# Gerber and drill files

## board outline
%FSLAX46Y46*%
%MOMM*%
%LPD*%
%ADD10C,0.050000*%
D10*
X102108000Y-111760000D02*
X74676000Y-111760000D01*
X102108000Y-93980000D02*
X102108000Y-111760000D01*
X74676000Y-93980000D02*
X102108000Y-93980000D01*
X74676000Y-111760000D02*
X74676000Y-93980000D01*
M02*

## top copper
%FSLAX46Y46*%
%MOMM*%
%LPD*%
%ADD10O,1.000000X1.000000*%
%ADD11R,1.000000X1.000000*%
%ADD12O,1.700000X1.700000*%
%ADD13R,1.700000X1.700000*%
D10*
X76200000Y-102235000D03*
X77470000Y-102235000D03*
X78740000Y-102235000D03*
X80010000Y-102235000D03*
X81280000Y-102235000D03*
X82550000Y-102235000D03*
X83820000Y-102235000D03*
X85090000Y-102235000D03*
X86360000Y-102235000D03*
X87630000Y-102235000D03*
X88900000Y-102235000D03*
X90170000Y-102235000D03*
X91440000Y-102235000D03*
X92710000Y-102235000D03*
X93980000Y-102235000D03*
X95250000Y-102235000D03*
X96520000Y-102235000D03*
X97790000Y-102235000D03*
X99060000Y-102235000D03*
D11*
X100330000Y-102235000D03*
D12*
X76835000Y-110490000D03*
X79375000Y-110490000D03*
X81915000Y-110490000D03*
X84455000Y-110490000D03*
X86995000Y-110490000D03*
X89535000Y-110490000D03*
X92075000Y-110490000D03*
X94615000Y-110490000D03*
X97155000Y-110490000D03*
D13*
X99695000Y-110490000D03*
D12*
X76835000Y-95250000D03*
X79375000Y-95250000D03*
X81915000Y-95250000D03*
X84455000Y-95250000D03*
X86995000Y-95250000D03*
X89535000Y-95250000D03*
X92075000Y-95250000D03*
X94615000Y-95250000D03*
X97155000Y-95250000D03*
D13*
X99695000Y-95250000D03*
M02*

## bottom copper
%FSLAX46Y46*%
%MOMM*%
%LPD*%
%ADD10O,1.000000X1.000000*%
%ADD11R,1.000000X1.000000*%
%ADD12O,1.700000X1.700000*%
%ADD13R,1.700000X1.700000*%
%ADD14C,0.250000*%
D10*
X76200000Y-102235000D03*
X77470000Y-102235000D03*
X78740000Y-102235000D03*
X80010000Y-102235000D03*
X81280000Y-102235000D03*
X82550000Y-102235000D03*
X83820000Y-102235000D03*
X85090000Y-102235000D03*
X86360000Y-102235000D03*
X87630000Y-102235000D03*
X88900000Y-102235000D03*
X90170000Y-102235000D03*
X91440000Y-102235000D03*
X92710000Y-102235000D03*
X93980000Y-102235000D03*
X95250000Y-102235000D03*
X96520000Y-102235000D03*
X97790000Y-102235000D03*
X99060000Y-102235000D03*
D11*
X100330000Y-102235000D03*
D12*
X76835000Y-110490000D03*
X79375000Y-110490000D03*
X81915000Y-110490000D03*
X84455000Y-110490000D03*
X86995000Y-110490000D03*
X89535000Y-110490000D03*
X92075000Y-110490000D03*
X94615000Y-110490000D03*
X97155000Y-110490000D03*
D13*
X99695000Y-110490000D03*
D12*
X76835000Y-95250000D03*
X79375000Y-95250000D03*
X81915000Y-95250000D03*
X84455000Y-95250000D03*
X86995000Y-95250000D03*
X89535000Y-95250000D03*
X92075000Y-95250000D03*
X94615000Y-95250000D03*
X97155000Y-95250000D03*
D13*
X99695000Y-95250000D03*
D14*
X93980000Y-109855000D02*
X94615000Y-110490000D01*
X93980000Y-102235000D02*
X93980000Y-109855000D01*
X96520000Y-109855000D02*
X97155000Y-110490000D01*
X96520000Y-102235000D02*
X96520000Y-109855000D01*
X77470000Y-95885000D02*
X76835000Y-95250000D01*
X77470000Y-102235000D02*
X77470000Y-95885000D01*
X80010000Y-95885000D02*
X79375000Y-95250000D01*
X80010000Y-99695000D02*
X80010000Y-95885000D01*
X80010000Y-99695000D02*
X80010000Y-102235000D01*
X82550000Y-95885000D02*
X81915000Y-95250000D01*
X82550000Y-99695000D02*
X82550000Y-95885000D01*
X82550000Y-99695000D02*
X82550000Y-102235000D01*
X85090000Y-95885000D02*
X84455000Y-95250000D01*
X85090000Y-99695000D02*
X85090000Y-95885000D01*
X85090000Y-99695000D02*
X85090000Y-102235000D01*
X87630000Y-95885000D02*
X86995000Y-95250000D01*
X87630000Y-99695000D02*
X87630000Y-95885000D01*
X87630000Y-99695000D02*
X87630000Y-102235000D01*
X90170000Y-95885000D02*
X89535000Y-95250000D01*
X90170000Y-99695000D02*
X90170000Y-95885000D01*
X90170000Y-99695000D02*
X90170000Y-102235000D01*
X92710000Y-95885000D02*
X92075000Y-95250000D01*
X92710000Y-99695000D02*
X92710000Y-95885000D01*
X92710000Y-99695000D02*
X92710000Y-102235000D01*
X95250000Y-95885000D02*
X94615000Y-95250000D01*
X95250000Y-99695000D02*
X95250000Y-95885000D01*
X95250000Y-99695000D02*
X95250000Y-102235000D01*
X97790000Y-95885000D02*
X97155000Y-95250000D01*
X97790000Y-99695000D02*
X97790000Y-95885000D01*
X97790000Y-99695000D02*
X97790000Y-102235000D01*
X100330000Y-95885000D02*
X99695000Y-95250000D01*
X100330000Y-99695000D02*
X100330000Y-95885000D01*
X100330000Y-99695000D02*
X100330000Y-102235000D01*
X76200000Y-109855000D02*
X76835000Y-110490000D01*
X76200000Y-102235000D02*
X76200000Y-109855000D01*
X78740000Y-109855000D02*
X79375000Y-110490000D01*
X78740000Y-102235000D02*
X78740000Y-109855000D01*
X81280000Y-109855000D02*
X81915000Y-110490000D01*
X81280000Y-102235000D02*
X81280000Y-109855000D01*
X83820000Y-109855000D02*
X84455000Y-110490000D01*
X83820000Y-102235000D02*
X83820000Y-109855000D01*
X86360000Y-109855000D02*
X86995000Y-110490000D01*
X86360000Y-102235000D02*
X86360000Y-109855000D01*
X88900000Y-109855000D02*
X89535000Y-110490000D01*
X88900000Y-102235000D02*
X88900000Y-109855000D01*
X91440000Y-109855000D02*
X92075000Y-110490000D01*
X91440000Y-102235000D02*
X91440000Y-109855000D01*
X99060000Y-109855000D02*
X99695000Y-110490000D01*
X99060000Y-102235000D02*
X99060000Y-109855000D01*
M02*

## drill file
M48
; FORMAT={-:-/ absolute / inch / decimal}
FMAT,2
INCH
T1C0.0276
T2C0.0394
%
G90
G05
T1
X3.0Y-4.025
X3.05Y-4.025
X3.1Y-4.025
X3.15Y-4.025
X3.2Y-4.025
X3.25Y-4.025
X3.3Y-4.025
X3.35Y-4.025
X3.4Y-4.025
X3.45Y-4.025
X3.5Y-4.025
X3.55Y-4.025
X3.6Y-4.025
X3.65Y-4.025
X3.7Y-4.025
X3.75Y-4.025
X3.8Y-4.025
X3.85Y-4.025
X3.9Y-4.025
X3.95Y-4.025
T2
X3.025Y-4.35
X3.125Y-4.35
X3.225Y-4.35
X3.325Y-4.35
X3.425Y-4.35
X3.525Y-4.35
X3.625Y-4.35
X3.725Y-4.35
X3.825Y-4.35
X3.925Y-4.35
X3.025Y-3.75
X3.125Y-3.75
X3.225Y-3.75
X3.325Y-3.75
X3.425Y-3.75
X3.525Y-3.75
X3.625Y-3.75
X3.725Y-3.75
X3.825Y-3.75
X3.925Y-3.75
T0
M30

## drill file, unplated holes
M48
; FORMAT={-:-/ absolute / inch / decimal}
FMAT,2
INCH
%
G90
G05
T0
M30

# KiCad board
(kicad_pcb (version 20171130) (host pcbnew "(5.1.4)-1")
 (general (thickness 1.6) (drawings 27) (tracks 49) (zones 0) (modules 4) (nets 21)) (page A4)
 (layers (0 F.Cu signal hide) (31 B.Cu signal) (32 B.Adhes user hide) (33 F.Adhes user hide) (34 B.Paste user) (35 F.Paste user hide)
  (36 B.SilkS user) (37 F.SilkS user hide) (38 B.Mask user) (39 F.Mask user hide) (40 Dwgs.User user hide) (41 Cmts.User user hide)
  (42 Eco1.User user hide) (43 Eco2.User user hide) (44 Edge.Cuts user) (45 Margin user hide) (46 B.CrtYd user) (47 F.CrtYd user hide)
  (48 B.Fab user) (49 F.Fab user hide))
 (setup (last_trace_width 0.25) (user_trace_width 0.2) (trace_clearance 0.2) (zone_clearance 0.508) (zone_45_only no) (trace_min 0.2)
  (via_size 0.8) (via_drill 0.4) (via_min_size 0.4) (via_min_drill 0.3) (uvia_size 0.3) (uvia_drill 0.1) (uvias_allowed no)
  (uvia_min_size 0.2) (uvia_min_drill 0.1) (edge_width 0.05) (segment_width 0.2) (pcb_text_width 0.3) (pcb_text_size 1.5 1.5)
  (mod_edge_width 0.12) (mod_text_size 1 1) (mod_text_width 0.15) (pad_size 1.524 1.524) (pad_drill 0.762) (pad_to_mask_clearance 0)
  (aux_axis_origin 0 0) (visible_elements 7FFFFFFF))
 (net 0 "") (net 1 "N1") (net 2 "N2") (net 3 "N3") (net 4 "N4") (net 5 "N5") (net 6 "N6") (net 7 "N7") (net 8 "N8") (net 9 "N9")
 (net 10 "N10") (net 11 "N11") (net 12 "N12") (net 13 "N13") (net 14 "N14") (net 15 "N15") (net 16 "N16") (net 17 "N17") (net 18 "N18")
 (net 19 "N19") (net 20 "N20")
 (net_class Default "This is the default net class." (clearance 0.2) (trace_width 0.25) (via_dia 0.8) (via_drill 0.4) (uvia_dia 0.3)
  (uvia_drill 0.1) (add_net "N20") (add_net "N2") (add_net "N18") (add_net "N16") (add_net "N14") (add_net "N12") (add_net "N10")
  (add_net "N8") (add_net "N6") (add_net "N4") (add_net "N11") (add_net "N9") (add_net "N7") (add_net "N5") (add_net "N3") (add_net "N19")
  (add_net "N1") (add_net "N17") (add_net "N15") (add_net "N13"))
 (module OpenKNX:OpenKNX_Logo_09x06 (layer B.Cu) (at 94.742 106.426 180)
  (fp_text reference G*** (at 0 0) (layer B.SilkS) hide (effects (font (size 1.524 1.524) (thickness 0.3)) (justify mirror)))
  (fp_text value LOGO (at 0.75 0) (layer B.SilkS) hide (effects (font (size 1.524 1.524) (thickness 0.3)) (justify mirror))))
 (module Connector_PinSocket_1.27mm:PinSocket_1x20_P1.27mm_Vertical (layer F.Cu) (at 100.33 102.235 270)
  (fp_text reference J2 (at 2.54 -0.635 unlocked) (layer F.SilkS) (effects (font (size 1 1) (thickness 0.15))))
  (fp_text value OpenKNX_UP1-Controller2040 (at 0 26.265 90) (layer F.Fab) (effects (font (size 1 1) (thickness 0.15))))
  (pad 20 thru_hole oval (at 0 24.13 270) (size 1 1) (drill 0.7) (layers *.Cu *.Mask) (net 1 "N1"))
  (pad 19 thru_hole oval (at 0 22.86 270) (size 1 1) (drill 0.7) (layers *.Cu *.Mask) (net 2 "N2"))
  (pad 18 thru_hole oval (at 0 21.59 270) (size 1 1) (drill 0.7) (layers *.Cu *.Mask) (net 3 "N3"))
  (pad 17 thru_hole oval (at 0 20.32 270) (size 1 1) (drill 0.7) (layers *.Cu *.Mask) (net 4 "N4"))
  (pad 16 thru_hole oval (at 0 19.05 270) (size 1 1) (drill 0.7) (layers *.Cu *.Mask) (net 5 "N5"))
  (pad 15 thru_hole oval (at 0 17.78 270) (size 1 1) (drill 0.7) (layers *.Cu *.Mask) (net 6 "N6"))
  (pad 14 thru_hole oval (at 0 16.51 270) (size 1 1) (drill 0.7) (layers *.Cu *.Mask) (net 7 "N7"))
  (pad 13 thru_hole oval (at 0 15.24 270) (size 1 1) (drill 0.7) (layers *.Cu *.Mask) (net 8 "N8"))
  (pad 12 thru_hole oval (at 0 13.97 270) (size 1 1) (drill 0.7) (layers *.Cu *.Mask) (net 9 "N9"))
  (pad 11 thru_hole oval (at 0 12.7 270) (size 1 1) (drill 0.7) (layers *.Cu *.Mask) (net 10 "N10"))
  (pad 10 thru_hole oval (at 0 11.43 270) (size 1 1) (drill 0.7) (layers *.Cu *.Mask) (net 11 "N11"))
  (pad 9 thru_hole oval (at 0 10.16 270) (size 1 1) (drill 0.7) (layers *.Cu *.Mask) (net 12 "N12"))
  (pad 8 thru_hole oval (at 0 8.89 270) (size 1 1) (drill 0.7) (layers *.Cu *.Mask) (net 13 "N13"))
  (pad 7 thru_hole oval (at 0 7.62 270) (size 1 1) (drill 0.7) (layers *.Cu *.Mask) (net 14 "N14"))
  (pad 6 thru_hole oval (at 0 6.35 270) (size 1 1) (drill 0.7) (layers *.Cu *.Mask) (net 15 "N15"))
  (pad 5 thru_hole oval (at 0 5.08 270) (size 1 1) (drill 0.7) (layers *.Cu *.Mask) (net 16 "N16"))
  (pad 4 thru_hole oval (at 0 3.81 270) (size 1 1) (drill 0.7) (layers *.Cu *.Mask) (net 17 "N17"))
  (pad 3 thru_hole oval (at 0 2.54 270) (size 1 1) (drill 0.7) (layers *.Cu *.Mask) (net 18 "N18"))
  (pad 2 thru_hole oval (at 0 1.27 270) (size 1 1) (drill 0.7) (layers *.Cu *.Mask) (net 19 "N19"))
  (pad 1 thru_hole rect (at 0 0 270) (size 1 1) (drill 0.7) (layers *.Cu *.Mask) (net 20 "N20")))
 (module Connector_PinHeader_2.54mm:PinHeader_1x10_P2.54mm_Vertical (layer B.Cu) (at 99.695 110.49 90)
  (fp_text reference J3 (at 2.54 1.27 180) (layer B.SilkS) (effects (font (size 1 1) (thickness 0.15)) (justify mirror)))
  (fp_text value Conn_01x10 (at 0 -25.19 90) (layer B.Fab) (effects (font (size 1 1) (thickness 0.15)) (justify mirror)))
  (pad 10 thru_hole oval (at 0 -22.86 90) (size 1.7 1.7) (drill 1) (layers *.Cu *.Mask) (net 1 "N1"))
  (pad 9 thru_hole oval (at 0 -20.32 90) (size 1.7 1.7) (drill 1) (layers *.Cu *.Mask) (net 3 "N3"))
  (pad 8 thru_hole oval (at 0 -17.78 90) (size 1.7 1.7) (drill 1) (layers *.Cu *.Mask) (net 5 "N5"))
  (pad 7 thru_hole oval (at 0 -15.24 90) (size 1.7 1.7) (drill 1) (layers *.Cu *.Mask) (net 7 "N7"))
  (pad 6 thru_hole oval (at 0 -12.7 90) (size 1.7 1.7) (drill 1) (layers *.Cu *.Mask) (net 9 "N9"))
  (pad 5 thru_hole oval (at 0 -10.16 90) (size 1.7 1.7) (drill 1) (layers *.Cu *.Mask) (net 11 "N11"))
  (pad 4 thru_hole oval (at 0 -7.62 90) (size 1.7 1.7) (drill 1) (layers *.Cu *.Mask) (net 13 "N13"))
  (pad 3 thru_hole oval (at 0 -5.08 90) (size 1.7 1.7) (drill 1) (layers *.Cu *.Mask) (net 15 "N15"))
  (pad 2 thru_hole oval (at 0 -2.54 90) (size 1.7 1.7) (drill 1) (layers *.Cu *.Mask) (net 17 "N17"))
  (pad 1 thru_hole rect (at 0 0 90) (size 1.7 1.7) (drill 1) (layers *.Cu *.Mask) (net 19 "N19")))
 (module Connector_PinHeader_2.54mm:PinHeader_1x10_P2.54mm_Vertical (layer B.Cu) (at 99.695 95.25 90)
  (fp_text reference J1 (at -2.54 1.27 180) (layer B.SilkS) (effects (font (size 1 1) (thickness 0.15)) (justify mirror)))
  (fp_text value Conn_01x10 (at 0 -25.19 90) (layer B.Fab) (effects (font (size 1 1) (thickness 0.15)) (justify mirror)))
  (pad 10 thru_hole oval (at 0 -22.86 90) (size 1.7 1.7) (drill 1) (layers *.Cu *.Mask) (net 2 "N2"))
  (pad 9 thru_hole oval (at 0 -20.32 90) (size 1.7 1.7) (drill 1) (layers *.Cu *.Mask) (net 4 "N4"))
  (pad 8 thru_hole oval (at 0 -17.78 90) (size 1.7 1.7) (drill 1) (layers *.Cu *.Mask) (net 6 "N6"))
  (pad 7 thru_hole oval (at 0 -15.24 90) (size 1.7 1.7) (drill 1) (layers *.Cu *.Mask) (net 8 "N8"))
  (pad 6 thru_hole oval (at 0 -12.7 90) (size 1.7 1.7) (drill 1) (layers *.Cu *.Mask) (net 10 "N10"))
  (pad 5 thru_hole oval (at 0 -10.16 90) (size 1.7 1.7) (drill 1) (layers *.Cu *.Mask) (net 12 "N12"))
  (pad 4 thru_hole oval (at 0 -7.62 90) (size 1.7 1.7) (drill 1) (layers *.Cu *.Mask) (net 14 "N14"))
  (pad 3 thru_hole oval (at 0 -5.08 90) (size 1.7 1.7) (drill 1) (layers *.Cu *.Mask) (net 16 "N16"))
  (pad 2 thru_hole oval (at 0 -2.54 90) (size 1.7 1.7) (drill 1) (layers *.Cu *.Mask) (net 18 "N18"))
  (pad 1 thru_hole rect (at 0 0 90) (size 1.7 1.7) (drill 1) (layers *.Cu *.Mask) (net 20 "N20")))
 (gr_line (start 102.108 111.76) (end 74.676 111.76) (layer Edge.Cuts) (width 0.05))
 (gr_line (start 102.108 93.98) (end 102.108 111.76) (layer Edge.Cuts) (width 0.05))
 (gr_line (start 74.676 93.98) (end 102.108 93.98) (layer Edge.Cuts) (width 0.05))
 (gr_line (start 74.676 111.76) (end 74.676 93.98) (layer Edge.Cuts) (width 0.05))
 (segment (start 93.98 109.855) (end 94.615 110.49) (width 0.25) (layer B.Cu) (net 15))
 (segment (start 93.98 102.235) (end 93.98 109.855) (width 0.25) (layer B.Cu) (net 15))
 (segment (start 96.52 109.855) (end 97.155 110.49) (width 0.25) (layer B.Cu) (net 17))
 (segment (start 96.52 102.235) (end 96.52 109.855) (width 0.25) (layer B.Cu) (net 17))
 (segment (start 77.47 95.885) (end 76.835 95.25) (width 0.25) (layer B.Cu) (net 2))
 (segment (start 77.47 102.235) (end 77.47 95.885) (width 0.25) (layer B.Cu) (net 2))
 (segment (start 80.01 95.885) (end 79.375 95.25) (width 0.25) (layer B.Cu) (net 4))
 (segment (start 80.01 99.695) (end 80.01 95.885) (width 0.25) (layer B.Cu) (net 4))
 (segment (start 80.01 99.695) (end 80.01 102.235) (width 0.25) (layer B.Cu) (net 4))
 (segment (start 82.55 95.885) (end 81.915 95.25) (width 0.25) (layer B.Cu) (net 6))
 (segment (start 82.55 99.695) (end 82.55 95.885) (width 0.25) (layer B.Cu) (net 6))
 (segment (start 82.55 99.695) (end 82.55 102.235) (width 0.25) (layer B.Cu) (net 6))
 (segment (start 85.09 95.885) (end 84.455 95.25) (width 0.25) (layer B.Cu) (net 8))
 (segment (start 85.09 99.695) (end 85.09 95.885) (width 0.25) (layer B.Cu) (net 8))
 (segment (start 85.09 99.695) (end 85.09 102.235) (width 0.25) (layer B.Cu) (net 8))
 (segment (start 87.63 95.885) (end 86.995 95.25) (width 0.25) (layer B.Cu) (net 10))
 (segment (start 87.63 99.695) (end 87.63 95.885) (width 0.25) (layer B.Cu) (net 10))
 (segment (start 87.63 99.695) (end 87.63 102.235) (width 0.25) (layer B.Cu) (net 10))
 (segment (start 90.17 95.885) (end 89.535 95.25) (width 0.25) (layer B.Cu) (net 12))
 (segment (start 90.17 99.695) (end 90.17 95.885) (width 0.25) (layer B.Cu) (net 12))
 (segment (start 90.17 99.695) (end 90.17 102.235) (width 0.25) (layer B.Cu) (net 12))
 (segment (start 92.71 95.885) (end 92.075 95.25) (width 0.25) (layer B.Cu) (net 14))
 (segment (start 92.71 99.695) (end 92.71 95.885) (width 0.25) (layer B.Cu) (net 14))
 (segment (start 92.71 99.695) (end 92.71 102.235) (width 0.25) (layer B.Cu) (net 14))
 (segment (start 95.25 95.885) (end 94.615 95.25) (width 0.25) (layer B.Cu) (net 16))
 (segment (start 95.25 99.695) (end 95.25 95.885) (width 0.25) (layer B.Cu) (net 16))
 (segment (start 95.25 99.695) (end 95.25 102.235) (width 0.25) (layer B.Cu) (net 16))
 (segment (start 97.79 95.885) (end 97.155 95.25) (width 0.25) (layer B.Cu) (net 18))
 (segment (start 97.79 99.695) (end 97.79 95.885) (width 0.25) (layer B.Cu) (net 18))
 (segment (start 97.79 99.695) (end 97.79 102.235) (width 0.25) (layer B.Cu) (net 18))
 (segment (start 100.33 95.885) (end 99.695 95.25) (width 0.25) (layer B.Cu) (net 20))
 (segment (start 100.33 99.695) (end 100.33 95.885) (width 0.25) (layer B.Cu) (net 20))
 (segment (start 100.33 99.695) (end 100.33 102.235) (width 0.25) (layer B.Cu) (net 20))
 (segment (start 76.2 109.855) (end 76.835 110.49) (width 0.25) (layer B.Cu) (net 1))
 (segment (start 76.2 102.235) (end 76.2 109.855) (width 0.25) (layer B.Cu) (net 1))
 (segment (start 78.74 109.855) (end 79.375 110.49) (width 0.25) (layer B.Cu) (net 3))
 (segment (start 78.74 102.235) (end 78.74 109.855) (width 0.25) (layer B.Cu) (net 3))
 (segment (start 81.28 109.855) (end 81.915 110.49) (width 0.25) (layer B.Cu) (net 5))
 (segment (start 81.28 102.235) (end 81.28 109.855) (width 0.25) (layer B.Cu) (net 5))
 (segment (start 83.82 109.855) (end 84.455 110.49) (width 0.25) (layer B.Cu) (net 7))
 (segment (start 83.82 102.235) (end 83.82 109.855) (width 0.25) (layer B.Cu) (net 7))
 (segment (start 86.36 109.855) (end 86.995 110.49) (width 0.25) (layer B.Cu) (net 9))
 (segment (start 86.36 102.235) (end 86.36 109.855) (width 0.25) (layer B.Cu) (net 9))
 (segment (start 88.9 109.855) (end 89.535 110.49) (width 0.25) (layer B.Cu) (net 11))
 (segment (start 88.9 102.235) (end 88.9 109.855) (width 0.25) (layer B.Cu) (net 11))
 (segment (start 91.44 109.855) (end 92.075 110.49) (width 0.25) (layer B.Cu) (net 13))
 (segment (start 91.44 102.235) (end 91.44 109.855) (width 0.25) (layer B.Cu) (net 13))
 (segment (start 99.06 109.855) (end 99.695 110.49) (width 0.25) (layer B.Cu) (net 19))
 (segment (start 99.06 102.235) (end 99.06 109.855) (width 0.25) (layer B.Cu) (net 19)))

